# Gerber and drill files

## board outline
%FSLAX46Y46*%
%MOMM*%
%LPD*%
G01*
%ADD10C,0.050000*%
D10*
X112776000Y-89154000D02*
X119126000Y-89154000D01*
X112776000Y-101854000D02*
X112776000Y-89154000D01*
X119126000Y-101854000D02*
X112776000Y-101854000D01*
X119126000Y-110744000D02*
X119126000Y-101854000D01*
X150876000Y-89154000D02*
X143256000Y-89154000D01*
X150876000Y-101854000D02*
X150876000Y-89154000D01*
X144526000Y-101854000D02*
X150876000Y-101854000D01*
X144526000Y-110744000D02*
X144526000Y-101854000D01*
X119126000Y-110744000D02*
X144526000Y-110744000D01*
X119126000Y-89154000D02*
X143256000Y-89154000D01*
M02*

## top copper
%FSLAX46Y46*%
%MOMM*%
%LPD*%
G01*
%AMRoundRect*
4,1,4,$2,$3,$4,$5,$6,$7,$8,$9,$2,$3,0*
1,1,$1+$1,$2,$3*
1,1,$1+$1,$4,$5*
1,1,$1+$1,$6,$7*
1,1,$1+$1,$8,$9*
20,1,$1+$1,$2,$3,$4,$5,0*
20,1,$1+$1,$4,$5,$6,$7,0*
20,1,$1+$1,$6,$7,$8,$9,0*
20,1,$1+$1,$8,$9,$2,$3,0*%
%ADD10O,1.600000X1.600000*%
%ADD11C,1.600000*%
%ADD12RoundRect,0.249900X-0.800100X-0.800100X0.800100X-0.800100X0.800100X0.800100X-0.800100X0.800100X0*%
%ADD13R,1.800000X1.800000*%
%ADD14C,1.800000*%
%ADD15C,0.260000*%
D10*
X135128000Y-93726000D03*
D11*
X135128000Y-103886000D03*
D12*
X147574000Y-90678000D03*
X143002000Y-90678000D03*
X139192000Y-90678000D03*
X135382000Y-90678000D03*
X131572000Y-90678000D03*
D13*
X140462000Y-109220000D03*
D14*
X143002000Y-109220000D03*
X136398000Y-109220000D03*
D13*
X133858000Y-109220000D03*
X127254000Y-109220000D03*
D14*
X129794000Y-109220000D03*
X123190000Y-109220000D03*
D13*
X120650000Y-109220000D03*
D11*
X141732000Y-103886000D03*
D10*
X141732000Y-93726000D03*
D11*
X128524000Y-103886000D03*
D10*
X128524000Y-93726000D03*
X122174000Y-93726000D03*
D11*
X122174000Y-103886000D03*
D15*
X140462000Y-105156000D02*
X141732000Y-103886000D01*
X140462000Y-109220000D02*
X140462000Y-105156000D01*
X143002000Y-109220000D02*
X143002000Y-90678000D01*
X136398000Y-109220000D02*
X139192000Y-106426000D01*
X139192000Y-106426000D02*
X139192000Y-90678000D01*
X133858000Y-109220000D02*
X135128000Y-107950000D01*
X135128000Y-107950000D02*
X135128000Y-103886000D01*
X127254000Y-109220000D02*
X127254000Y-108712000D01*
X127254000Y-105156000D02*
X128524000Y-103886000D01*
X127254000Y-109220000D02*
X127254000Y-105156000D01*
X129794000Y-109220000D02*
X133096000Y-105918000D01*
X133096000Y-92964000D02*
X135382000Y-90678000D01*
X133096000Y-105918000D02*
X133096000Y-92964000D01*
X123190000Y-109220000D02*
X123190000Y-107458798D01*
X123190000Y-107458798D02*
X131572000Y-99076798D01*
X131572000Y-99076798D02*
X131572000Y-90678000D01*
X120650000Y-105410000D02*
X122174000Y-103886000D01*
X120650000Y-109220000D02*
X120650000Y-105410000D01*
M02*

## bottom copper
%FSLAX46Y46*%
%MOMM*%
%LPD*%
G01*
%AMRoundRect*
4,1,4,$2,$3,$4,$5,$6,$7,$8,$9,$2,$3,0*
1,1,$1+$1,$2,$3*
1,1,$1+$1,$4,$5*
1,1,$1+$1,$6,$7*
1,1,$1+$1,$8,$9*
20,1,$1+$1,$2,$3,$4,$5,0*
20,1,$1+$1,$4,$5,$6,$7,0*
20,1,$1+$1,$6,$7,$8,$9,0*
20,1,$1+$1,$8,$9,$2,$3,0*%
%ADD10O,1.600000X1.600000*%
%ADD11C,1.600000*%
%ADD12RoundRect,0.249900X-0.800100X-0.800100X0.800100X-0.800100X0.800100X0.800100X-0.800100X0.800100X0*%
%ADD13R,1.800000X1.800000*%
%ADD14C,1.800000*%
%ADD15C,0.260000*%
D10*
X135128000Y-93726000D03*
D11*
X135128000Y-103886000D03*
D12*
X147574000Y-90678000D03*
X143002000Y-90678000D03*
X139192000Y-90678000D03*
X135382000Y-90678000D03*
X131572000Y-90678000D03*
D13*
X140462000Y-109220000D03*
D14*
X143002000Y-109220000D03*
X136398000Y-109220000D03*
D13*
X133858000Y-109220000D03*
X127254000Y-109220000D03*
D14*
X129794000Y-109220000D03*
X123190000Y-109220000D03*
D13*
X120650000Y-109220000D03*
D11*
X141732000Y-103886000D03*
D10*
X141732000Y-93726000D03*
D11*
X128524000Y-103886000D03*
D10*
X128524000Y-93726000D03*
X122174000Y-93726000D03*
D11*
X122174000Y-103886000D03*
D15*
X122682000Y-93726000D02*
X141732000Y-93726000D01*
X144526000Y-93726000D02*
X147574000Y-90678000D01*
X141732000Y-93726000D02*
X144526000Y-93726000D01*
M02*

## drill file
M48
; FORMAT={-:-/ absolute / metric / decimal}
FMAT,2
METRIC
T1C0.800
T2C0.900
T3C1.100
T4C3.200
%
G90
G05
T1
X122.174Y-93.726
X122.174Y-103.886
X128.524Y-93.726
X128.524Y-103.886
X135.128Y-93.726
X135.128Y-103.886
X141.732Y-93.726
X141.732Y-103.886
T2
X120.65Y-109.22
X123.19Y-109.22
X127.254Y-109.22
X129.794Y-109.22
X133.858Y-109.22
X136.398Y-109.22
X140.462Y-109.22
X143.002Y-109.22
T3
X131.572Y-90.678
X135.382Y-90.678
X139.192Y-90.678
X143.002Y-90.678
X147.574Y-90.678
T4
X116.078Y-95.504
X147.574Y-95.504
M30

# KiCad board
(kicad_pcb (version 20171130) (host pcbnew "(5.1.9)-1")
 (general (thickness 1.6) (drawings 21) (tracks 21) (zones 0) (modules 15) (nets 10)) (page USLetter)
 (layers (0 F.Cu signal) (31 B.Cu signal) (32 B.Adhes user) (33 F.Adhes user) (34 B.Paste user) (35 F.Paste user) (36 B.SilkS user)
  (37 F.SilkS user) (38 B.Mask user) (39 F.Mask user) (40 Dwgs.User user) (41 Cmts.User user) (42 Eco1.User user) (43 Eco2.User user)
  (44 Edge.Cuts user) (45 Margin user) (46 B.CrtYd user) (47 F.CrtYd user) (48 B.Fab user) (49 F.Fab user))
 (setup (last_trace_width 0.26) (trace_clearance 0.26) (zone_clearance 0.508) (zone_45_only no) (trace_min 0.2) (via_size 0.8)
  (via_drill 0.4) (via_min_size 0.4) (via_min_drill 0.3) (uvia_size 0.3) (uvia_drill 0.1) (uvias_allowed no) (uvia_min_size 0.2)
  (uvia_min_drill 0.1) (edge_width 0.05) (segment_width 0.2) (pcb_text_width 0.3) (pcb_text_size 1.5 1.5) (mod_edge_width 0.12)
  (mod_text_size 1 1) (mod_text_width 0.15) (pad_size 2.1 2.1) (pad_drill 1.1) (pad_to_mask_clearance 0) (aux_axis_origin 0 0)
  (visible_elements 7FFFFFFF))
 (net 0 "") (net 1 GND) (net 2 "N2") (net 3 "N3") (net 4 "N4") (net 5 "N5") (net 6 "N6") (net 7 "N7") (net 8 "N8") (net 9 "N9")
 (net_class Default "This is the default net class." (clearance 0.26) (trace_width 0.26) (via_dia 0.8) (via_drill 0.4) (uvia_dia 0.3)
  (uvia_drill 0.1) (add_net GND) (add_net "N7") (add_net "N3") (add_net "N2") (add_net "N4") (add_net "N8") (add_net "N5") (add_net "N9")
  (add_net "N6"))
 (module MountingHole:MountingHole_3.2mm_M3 (layer F.Cu) (at 116.078 95.504)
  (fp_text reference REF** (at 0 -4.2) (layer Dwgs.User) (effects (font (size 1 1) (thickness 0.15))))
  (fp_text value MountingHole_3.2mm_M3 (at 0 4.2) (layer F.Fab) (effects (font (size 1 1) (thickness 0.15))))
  (pad 1 np_thru_hole circle (at 0 0) (size 3.2 3.2) (drill 3.2) (layers *.Cu *.Mask)))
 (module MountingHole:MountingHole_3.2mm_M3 (layer F.Cu) (at 147.574 95.504)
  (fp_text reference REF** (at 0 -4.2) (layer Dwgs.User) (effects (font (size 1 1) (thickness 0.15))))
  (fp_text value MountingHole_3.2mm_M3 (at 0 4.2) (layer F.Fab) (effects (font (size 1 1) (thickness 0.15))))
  (pad 1 np_thru_hole circle (at 0 0) (size 3.2 3.2) (drill 3.2) (layers *.Cu *.Mask)))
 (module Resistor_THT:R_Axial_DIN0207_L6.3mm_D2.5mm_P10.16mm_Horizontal (layer F.Cu) (at 135.128 103.886 90)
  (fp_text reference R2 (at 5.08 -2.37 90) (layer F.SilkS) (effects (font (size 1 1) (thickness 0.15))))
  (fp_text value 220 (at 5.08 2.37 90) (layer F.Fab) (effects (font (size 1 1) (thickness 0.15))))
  (pad 2 thru_hole oval (at 10.16 0 90) (size 1.6 1.6) (drill 0.8) (layers *.Cu *.Mask) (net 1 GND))
  (pad 1 thru_hole circle (at 0 0 90) (size 1.6 1.6) (drill 0.8) (layers *.Cu *.Mask) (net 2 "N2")))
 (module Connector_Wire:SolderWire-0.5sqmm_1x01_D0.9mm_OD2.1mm (layer F.Cu) (at 147.574 90.678)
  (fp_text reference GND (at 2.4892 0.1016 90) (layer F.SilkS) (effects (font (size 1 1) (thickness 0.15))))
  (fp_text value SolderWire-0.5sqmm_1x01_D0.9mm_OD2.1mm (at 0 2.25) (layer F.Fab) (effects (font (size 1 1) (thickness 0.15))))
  (pad 1 thru_hole roundrect (at 0 0) (size 2.1 2.1) (drill 1.1) (layers *.Cu *.Mask) (roundrect_rratio 0.119) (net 1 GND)))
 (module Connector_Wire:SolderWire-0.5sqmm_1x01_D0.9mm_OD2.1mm (layer F.Cu) (at 143.002 90.678)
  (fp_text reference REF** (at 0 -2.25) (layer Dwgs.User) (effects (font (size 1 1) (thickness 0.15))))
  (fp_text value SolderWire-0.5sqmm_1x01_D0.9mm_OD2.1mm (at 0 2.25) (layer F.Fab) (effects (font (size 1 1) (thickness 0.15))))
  (pad 1 thru_hole roundrect (at 0 0) (size 2.1 2.1) (drill 1.1) (layers *.Cu *.Mask) (roundrect_rratio 0.119) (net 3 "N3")))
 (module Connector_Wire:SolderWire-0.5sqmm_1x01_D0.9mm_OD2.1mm (layer F.Cu) (at 139.192 90.678)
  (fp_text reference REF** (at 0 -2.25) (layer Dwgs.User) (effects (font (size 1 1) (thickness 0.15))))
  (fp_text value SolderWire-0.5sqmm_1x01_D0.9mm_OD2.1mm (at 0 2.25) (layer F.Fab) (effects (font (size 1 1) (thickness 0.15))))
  (pad 1 thru_hole roundrect (at 0 0) (size 2.1 2.1) (drill 1.1) (layers *.Cu *.Mask) (roundrect_rratio 0.119) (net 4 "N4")))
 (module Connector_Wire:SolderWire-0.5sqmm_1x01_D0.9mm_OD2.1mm (layer F.Cu) (at 135.382 90.678)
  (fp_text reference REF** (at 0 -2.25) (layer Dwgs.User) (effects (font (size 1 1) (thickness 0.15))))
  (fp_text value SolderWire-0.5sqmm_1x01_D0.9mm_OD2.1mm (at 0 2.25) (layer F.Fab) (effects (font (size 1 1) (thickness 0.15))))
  (pad 1 thru_hole roundrect (at 0 0) (size 2.1 2.1) (drill 1.1) (layers *.Cu *.Mask) (roundrect_rratio 0.119) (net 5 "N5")))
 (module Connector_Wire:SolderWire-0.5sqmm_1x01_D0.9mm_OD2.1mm (layer F.Cu) (at 131.572 90.678)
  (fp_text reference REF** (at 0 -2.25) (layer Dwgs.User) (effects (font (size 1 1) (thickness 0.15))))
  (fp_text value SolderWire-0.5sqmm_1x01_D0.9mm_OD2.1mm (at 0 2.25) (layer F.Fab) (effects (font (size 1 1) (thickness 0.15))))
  (pad 1 thru_hole roundrect (at 0 0) (size 2.1 2.1) (drill 1.1) (layers *.Cu *.Mask) (roundrect_rratio 0.119) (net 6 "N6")))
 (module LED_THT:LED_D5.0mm (layer F.Cu) (at 140.462 109.22)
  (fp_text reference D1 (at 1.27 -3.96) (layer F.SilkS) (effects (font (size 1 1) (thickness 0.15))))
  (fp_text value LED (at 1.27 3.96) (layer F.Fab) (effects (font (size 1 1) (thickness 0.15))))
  (pad 1 thru_hole rect (at 0 0) (size 1.8 1.8) (drill 0.9) (layers *.Cu *.Mask) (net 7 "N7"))
  (pad 2 thru_hole circle (at 2.54 0) (size 1.8 1.8) (drill 0.9) (layers *.Cu *.Mask) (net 3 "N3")))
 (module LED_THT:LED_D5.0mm (layer F.Cu) (at 133.858 109.22)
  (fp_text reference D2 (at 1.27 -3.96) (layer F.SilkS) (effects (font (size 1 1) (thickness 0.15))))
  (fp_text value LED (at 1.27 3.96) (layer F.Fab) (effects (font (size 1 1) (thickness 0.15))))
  (pad 2 thru_hole circle (at 2.54 0) (size 1.8 1.8) (drill 0.9) (layers *.Cu *.Mask) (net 4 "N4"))
  (pad 1 thru_hole rect (at 0 0) (size 1.8 1.8) (drill 0.9) (layers *.Cu *.Mask) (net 2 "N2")))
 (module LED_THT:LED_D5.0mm (layer F.Cu) (at 127.254 109.22)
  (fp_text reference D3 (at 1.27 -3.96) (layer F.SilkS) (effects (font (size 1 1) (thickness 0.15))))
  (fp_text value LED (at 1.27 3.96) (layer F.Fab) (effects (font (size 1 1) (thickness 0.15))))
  (pad 1 thru_hole rect (at 0 0) (size 1.8 1.8) (drill 0.9) (layers *.Cu *.Mask) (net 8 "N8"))
  (pad 2 thru_hole circle (at 2.54 0) (size 1.8 1.8) (drill 0.9) (layers *.Cu *.Mask) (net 5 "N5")))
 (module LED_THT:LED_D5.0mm (layer F.Cu) (at 120.65 109.22)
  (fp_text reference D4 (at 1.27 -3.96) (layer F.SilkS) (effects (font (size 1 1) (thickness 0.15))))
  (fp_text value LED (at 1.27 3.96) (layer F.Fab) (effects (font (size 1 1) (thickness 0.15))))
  (pad 2 thru_hole circle (at 2.54 0) (size 1.8 1.8) (drill 0.9) (layers *.Cu *.Mask) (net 6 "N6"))
  (pad 1 thru_hole rect (at 0 0) (size 1.8 1.8) (drill 0.9) (layers *.Cu *.Mask) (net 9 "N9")))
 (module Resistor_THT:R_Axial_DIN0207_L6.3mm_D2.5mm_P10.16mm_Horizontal (layer F.Cu) (at 141.732 103.886 90)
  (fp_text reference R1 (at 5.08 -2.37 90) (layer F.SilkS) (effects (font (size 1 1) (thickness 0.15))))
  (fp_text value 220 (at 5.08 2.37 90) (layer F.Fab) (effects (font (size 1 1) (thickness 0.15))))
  (pad 1 thru_hole circle (at 0 0 90) (size 1.6 1.6) (drill 0.8) (layers *.Cu *.Mask) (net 7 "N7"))
  (pad 2 thru_hole oval (at 10.16 0 90) (size 1.6 1.6) (drill 0.8) (layers *.Cu *.Mask) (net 1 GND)))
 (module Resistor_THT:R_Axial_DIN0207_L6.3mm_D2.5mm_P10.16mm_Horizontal (layer F.Cu) (at 128.524 103.886 90)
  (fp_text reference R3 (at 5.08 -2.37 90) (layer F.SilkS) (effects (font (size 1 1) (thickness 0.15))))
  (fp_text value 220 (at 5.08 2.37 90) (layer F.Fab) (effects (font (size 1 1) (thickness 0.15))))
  (pad 1 thru_hole circle (at 0 0 90) (size 1.6 1.6) (drill 0.8) (layers *.Cu *.Mask) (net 8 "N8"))
  (pad 2 thru_hole oval (at 10.16 0 90) (size 1.6 1.6) (drill 0.8) (layers *.Cu *.Mask) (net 1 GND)))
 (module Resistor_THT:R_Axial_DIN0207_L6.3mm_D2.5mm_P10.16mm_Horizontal (layer F.Cu) (at 122.174 103.886 90)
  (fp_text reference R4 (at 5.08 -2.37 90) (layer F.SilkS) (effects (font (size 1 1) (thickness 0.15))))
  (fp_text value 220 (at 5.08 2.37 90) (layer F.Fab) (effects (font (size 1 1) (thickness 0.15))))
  (pad 2 thru_hole oval (at 10.16 0 90) (size 1.6 1.6) (drill 0.8) (layers *.Cu *.Mask) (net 1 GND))
  (pad 1 thru_hole circle (at 0 0 90) (size 1.6 1.6) (drill 0.8) (layers *.Cu *.Mask) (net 9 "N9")))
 (gr_line (start 112.776 89.154) (end 119.126 89.154) (layer Edge.Cuts) (width 0.05))
 (gr_line (start 112.776 101.854) (end 112.776 89.154) (layer Edge.Cuts) (width 0.05))
 (gr_line (start 119.126 101.854) (end 112.776 101.854) (layer Edge.Cuts) (width 0.05))
 (gr_line (start 119.126 110.744) (end 119.126 101.854) (layer Edge.Cuts) (width 0.05))
 (gr_line (start 150.876 89.154) (end 143.256 89.154) (layer Edge.Cuts) (width 0.05))
 (gr_line (start 150.876 101.854) (end 150.876 89.154) (layer Edge.Cuts) (width 0.05))
 (gr_line (start 144.526 101.854) (end 150.876 101.854) (layer Edge.Cuts) (width 0.05))
 (gr_line (start 144.526 110.744) (end 144.526 101.854) (layer Edge.Cuts) (width 0.05))
 (gr_line (start 119.126 110.744) (end 144.526 110.744) (layer Edge.Cuts) (width 0.05))
 (gr_line (start 119.126 89.154) (end 143.256 89.154) (layer Edge.Cuts) (width 0.05))
 (segment (start 140.462 105.156) (end 141.732 103.886) (width 0.26) (layer F.Cu) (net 7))
 (segment (start 140.462 109.22) (end 140.462 105.156) (width 0.26) (layer F.Cu) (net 7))
 (segment (start 143.002 109.22) (end 143.002 90.678) (width 0.26) (layer F.Cu) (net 3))
 (segment (start 136.398 109.22) (end 139.192 106.426) (width 0.26) (layer F.Cu) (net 4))
 (segment (start 139.192 106.426) (end 139.192 90.678) (width 0.26) (layer F.Cu) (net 4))
 (segment (start 133.858 109.22) (end 135.128 107.95) (width 0.26) (layer F.Cu) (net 2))
 (segment (start 135.128 107.95) (end 135.128 103.886) (width 0.26) (layer F.Cu) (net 2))
 (segment (start 127.254 109.22) (end 127.254 108.712) (width 0.26) (layer F.Cu) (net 8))
 (segment (start 127.254 105.156) (end 128.524 103.886) (width 0.26) (layer F.Cu) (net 8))
 (segment (start 127.254 109.22) (end 127.254 105.156) (width 0.26) (layer F.Cu) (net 8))
 (segment (start 129.794 109.22) (end 133.096 105.918) (width 0.26) (layer F.Cu) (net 5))
 (segment (start 133.096 92.964) (end 135.382 90.678) (width 0.26) (layer F.Cu) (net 5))
 (segment (start 133.096 105.918) (end 133.096 92.964) (width 0.26) (layer F.Cu) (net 5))
 (segment (start 123.19 109.22) (end 123.19 107.458798) (width 0.26) (layer F.Cu) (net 6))
 (segment (start 123.19 107.458798) (end 131.572 99.076798) (width 0.26) (layer F.Cu) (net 6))
 (segment (start 131.572 99.076798) (end 131.572 90.678) (width 0.26) (layer F.Cu) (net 6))
 (segment (start 120.65 105.41) (end 122.174 103.886) (width 0.26) (layer F.Cu) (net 9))
 (segment (start 120.65 109.22) (end 120.65 105.41) (width 0.26) (layer F.Cu) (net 9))
 (segment (start 122.682 93.726) (end 141.732 93.726) (width 0.26) (layer B.Cu) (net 1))
 (segment (start 144.526 93.726) (end 147.574 90.678) (width 0.26) (layer B.Cu) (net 1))
 (segment (start 141.732 93.726) (end 144.526 93.726) (width 0.26) (layer B.Cu) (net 1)))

